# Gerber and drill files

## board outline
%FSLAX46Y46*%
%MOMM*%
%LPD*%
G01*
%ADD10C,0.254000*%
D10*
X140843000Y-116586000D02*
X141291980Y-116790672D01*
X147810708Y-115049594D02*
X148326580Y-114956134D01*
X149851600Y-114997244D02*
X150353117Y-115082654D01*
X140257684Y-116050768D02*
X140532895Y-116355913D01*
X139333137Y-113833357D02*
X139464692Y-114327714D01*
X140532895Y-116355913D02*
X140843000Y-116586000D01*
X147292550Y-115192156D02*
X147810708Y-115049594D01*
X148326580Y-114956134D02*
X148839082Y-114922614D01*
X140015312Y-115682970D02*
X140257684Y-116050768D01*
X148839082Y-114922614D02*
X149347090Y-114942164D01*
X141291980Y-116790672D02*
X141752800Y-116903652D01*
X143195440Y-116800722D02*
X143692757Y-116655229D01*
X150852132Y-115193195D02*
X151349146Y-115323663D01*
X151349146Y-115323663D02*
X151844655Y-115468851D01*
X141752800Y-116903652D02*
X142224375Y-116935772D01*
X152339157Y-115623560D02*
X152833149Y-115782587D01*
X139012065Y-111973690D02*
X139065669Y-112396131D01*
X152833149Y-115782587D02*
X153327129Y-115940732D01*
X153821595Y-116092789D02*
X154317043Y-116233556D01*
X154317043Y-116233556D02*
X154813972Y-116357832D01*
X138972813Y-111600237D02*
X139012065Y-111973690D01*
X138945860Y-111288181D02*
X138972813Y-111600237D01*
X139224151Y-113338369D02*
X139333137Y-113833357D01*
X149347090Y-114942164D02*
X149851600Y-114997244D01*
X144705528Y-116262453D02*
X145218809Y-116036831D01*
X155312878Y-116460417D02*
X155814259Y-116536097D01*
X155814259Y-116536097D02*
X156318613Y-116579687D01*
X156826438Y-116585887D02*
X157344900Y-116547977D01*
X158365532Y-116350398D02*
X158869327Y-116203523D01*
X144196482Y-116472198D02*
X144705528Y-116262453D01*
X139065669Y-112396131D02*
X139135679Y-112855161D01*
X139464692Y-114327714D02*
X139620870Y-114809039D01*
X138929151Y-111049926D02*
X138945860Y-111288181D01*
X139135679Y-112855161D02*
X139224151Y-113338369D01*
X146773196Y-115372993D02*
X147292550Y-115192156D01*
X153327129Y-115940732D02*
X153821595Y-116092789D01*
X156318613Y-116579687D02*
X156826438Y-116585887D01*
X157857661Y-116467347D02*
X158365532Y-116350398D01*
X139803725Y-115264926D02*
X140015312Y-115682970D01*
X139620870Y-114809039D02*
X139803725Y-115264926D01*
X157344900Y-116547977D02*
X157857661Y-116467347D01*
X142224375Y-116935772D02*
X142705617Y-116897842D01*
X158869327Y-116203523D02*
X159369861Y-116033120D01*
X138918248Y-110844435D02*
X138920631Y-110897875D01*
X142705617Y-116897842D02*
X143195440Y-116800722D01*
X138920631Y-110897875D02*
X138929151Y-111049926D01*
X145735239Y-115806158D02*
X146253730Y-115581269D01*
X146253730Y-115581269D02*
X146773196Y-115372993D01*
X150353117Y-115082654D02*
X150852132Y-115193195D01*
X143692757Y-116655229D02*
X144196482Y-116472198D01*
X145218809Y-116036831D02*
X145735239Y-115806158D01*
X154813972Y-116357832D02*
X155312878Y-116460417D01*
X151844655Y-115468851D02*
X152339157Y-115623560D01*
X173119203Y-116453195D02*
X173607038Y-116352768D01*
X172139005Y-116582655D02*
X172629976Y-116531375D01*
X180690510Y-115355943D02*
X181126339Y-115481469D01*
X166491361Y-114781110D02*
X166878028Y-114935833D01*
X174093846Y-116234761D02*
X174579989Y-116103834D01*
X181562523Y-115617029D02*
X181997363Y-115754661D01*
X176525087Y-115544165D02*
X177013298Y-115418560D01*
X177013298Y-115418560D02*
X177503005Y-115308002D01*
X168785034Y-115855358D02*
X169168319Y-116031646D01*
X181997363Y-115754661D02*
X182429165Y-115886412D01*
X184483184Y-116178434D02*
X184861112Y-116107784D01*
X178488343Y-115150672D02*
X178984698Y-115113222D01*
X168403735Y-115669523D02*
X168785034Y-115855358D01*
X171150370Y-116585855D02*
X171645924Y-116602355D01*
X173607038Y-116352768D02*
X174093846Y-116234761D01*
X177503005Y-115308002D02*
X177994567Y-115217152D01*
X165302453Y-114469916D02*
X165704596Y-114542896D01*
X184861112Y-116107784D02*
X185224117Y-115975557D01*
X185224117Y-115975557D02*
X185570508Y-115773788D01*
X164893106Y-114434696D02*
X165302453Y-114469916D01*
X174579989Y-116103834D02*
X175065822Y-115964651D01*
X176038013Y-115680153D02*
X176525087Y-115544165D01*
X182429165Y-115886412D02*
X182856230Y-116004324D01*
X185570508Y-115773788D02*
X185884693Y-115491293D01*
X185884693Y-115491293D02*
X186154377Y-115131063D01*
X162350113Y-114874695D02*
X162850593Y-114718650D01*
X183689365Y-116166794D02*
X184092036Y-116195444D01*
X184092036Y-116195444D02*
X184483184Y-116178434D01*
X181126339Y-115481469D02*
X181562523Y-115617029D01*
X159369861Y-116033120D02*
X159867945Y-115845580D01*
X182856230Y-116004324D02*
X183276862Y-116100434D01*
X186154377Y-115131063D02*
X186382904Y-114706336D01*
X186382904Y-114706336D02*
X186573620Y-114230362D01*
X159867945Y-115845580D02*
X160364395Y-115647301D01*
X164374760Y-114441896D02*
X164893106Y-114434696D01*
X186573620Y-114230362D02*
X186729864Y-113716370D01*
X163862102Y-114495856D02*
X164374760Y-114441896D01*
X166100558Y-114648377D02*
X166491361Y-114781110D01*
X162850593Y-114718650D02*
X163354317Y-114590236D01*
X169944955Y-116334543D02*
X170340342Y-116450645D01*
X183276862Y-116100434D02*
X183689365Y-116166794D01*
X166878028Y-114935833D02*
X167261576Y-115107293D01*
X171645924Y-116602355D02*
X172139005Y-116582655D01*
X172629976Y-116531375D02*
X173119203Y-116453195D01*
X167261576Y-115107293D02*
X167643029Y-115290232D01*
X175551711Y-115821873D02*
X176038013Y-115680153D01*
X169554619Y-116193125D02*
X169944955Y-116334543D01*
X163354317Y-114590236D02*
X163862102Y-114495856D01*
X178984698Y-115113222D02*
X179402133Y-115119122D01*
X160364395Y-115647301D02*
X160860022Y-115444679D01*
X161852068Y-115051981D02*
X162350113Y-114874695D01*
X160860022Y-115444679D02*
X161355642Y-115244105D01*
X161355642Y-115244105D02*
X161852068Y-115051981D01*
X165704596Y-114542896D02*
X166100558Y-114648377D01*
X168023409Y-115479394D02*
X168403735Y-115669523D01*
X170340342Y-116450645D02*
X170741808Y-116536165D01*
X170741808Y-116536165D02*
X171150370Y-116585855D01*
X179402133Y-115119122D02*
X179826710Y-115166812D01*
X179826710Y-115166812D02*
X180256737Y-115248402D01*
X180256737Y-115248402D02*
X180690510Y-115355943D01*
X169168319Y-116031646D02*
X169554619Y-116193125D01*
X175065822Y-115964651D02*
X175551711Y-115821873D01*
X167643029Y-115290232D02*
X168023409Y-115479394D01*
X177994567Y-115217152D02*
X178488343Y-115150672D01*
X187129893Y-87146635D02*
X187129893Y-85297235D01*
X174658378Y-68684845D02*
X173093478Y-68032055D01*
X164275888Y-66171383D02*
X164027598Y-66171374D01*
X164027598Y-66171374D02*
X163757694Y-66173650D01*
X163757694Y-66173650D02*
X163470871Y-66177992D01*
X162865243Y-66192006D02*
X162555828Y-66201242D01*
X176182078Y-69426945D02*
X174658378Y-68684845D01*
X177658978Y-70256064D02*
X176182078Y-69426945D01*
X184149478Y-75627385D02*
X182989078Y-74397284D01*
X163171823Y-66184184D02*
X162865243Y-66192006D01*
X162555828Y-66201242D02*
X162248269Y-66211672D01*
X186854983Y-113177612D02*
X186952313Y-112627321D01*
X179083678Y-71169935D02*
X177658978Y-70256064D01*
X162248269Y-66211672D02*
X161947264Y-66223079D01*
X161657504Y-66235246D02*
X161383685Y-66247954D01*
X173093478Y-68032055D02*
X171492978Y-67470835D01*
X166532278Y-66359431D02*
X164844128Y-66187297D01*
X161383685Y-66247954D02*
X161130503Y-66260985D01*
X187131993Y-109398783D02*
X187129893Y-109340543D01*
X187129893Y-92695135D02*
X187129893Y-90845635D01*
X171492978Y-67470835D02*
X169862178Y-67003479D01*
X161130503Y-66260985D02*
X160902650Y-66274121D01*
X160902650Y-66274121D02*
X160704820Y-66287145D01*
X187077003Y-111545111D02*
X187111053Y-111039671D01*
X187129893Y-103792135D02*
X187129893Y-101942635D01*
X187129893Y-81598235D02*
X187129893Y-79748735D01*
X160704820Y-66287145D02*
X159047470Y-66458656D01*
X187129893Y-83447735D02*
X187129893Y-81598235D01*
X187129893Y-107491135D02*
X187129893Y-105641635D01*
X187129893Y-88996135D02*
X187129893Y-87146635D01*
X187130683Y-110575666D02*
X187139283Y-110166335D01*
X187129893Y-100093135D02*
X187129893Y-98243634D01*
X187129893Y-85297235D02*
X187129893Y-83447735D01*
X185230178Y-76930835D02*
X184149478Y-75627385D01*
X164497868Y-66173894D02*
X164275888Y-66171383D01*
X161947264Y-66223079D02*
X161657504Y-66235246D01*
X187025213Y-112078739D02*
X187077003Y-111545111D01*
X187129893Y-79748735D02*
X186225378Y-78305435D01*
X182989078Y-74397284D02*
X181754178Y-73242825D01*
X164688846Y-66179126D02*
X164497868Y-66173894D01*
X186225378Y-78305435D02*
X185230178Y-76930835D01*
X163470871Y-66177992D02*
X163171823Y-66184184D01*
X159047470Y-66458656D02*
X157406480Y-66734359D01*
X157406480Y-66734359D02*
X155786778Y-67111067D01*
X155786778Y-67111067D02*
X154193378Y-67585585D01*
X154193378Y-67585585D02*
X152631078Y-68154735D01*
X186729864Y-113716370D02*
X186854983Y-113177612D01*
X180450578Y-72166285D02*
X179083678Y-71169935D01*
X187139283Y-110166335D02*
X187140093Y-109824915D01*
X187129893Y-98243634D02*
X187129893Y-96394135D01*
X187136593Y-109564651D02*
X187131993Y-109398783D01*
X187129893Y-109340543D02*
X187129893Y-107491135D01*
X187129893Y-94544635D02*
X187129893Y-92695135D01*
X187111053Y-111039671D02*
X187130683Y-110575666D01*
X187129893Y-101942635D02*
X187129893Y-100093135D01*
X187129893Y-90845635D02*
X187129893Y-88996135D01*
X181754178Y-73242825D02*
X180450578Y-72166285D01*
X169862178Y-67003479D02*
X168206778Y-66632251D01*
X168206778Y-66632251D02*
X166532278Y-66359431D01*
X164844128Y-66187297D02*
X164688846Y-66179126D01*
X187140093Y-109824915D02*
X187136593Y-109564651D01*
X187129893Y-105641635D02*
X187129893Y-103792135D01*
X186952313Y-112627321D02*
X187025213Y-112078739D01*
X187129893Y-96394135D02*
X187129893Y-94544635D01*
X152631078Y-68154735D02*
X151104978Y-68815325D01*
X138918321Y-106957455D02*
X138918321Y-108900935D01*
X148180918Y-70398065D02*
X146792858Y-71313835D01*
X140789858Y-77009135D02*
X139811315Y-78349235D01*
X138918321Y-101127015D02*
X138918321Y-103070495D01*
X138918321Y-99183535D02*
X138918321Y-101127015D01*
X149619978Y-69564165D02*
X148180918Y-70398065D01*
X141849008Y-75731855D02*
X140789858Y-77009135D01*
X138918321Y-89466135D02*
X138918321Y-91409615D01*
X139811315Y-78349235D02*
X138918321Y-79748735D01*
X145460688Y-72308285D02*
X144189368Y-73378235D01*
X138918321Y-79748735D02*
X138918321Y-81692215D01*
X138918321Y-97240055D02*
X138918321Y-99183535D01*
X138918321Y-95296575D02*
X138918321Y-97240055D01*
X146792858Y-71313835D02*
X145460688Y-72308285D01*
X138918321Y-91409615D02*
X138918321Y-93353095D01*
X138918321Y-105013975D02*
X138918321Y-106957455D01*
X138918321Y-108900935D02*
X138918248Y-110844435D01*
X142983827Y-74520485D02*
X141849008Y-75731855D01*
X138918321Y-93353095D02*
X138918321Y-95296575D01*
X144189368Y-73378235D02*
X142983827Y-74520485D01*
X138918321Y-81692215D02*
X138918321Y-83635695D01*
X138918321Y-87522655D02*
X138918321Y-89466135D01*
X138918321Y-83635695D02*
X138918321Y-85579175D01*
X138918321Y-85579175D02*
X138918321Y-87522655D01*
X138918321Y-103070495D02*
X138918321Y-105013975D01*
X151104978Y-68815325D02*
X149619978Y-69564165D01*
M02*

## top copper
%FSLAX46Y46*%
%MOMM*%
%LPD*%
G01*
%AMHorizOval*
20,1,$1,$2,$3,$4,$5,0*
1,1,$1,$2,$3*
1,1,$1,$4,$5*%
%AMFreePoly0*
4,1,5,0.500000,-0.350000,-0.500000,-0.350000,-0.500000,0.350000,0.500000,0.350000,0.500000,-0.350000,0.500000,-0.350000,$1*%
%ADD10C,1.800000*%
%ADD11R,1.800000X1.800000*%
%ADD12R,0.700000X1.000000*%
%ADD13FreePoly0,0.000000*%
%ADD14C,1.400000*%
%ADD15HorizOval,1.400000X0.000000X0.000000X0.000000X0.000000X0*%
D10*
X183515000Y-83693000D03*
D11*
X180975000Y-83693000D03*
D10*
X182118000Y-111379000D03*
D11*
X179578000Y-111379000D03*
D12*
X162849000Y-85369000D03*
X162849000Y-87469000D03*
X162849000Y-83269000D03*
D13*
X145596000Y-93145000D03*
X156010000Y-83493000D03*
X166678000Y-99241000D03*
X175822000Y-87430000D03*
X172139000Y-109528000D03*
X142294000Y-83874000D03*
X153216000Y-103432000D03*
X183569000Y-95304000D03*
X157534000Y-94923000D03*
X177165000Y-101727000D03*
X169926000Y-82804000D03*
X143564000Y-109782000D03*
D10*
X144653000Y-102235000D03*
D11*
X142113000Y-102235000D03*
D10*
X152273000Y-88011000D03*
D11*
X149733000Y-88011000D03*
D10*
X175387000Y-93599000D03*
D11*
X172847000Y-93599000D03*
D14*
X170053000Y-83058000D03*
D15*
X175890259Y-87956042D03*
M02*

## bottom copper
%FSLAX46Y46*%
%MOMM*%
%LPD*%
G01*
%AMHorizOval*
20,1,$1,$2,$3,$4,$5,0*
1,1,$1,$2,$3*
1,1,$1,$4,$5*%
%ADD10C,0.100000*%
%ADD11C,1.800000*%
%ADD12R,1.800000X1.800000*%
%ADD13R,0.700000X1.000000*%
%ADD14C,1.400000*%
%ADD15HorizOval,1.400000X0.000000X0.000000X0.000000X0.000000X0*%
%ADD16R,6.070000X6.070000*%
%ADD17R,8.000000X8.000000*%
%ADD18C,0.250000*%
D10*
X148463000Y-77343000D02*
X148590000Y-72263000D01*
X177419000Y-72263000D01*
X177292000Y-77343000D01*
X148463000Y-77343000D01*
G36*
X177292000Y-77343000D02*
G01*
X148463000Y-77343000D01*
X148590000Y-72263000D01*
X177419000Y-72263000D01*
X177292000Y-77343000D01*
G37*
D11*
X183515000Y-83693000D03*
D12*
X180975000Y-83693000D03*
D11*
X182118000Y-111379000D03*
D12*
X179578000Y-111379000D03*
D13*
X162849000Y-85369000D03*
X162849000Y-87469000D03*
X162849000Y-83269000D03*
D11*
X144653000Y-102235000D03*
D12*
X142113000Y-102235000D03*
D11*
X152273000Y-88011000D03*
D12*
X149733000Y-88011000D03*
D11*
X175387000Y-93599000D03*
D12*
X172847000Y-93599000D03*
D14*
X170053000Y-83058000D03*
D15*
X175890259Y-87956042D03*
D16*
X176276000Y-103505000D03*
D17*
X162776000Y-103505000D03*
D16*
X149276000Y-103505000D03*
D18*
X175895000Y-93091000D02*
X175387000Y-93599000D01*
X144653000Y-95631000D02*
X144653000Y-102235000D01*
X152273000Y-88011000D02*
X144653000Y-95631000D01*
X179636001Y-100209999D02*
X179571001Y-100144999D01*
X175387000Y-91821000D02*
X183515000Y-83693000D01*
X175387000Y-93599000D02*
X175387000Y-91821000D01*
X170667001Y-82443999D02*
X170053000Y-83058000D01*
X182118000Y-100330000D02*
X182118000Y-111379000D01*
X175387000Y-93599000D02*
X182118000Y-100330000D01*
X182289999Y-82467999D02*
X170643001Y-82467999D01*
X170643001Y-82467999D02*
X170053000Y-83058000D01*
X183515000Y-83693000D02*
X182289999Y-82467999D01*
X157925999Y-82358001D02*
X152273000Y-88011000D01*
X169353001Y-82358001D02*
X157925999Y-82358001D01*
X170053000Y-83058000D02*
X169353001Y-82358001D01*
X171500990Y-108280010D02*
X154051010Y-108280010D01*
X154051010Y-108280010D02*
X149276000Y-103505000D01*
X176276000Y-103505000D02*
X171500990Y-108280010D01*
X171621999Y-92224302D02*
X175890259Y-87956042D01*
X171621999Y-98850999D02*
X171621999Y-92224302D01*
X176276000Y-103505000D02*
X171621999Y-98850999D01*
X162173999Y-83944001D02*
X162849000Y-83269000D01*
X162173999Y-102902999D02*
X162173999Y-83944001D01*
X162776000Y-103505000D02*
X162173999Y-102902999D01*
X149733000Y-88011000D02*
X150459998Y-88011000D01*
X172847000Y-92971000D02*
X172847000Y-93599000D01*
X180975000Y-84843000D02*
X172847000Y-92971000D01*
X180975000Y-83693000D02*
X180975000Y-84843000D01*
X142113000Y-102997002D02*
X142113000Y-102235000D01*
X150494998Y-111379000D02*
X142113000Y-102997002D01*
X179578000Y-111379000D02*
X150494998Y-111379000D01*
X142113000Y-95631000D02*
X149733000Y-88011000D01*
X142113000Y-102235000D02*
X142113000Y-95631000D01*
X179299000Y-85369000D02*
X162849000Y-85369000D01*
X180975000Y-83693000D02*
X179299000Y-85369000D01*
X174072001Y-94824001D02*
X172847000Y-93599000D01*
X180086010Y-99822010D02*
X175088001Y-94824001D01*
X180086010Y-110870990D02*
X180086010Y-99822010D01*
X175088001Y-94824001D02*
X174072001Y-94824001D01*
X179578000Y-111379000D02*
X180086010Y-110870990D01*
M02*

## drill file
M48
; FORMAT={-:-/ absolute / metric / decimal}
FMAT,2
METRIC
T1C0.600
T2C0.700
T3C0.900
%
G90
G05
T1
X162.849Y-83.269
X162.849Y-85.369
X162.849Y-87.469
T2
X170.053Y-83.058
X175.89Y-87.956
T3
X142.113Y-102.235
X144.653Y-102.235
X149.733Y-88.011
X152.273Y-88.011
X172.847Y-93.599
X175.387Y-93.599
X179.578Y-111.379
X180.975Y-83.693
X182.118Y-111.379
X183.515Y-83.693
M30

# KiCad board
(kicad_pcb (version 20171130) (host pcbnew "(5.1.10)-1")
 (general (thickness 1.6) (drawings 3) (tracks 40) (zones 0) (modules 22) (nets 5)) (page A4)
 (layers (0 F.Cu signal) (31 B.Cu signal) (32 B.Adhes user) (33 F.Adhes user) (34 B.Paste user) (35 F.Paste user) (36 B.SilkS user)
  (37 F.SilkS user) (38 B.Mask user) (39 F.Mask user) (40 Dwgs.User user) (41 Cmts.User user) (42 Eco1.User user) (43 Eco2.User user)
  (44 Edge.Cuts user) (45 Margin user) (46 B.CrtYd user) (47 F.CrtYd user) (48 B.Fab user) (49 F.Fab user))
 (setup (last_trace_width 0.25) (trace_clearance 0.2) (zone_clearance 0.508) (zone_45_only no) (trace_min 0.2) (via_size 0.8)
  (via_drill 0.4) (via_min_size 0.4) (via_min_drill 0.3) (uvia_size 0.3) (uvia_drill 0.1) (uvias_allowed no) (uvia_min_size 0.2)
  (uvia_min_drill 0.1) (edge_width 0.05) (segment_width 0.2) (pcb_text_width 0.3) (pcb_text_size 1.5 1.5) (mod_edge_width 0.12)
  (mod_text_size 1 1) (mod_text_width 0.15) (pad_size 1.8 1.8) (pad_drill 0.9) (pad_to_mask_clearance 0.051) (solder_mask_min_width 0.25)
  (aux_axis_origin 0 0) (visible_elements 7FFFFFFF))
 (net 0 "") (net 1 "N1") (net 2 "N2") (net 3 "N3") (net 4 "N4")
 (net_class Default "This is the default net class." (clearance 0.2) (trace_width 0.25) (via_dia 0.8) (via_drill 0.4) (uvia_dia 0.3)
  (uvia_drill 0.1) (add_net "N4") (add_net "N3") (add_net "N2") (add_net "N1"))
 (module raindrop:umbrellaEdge (layer F.Cu) (at 162.687 92.456)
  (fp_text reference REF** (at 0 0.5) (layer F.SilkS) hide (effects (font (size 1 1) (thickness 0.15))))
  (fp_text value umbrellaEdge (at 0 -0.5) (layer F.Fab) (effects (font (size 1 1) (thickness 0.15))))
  (fp_line (start -21.844 24.13) (end -21.39502 24.334672) (layer Edge.Cuts) (width 0.254))
  (fp_line (start -14.876292 22.593594) (end -14.36042 22.500134) (layer Edge.Cuts) (width 0.254))
  (fp_line (start -12.8354 22.541244) (end -12.333883 22.626654) (layer Edge.Cuts) (width 0.254))
  (fp_line (start -22.429316 23.594768) (end -22.154105 23.899913) (layer Edge.Cuts) (width 0.254))
  (fp_line (start -23.353863 21.377357) (end -23.222308 21.871714) (layer Edge.Cuts) (width 0.254))
  (fp_line (start -22.154105 23.899913) (end -21.844 24.13) (layer Edge.Cuts) (width 0.254))
  (fp_line (start -15.39445 22.736156) (end -14.876292 22.593594) (layer Edge.Cuts) (width 0.254))
  (fp_line (start -14.36042 22.500134) (end -13.847918 22.466614) (layer Edge.Cuts) (width 0.254))
  (fp_line (start -22.671688 23.22697) (end -22.429316 23.594768) (layer Edge.Cuts) (width 0.254))
  (fp_line (start -13.847918 22.466614) (end -13.33991 22.486164) (layer Edge.Cuts) (width 0.254))
  (fp_line (start -21.39502 24.334672) (end -20.9342 24.447652) (layer Edge.Cuts) (width 0.254))
  (fp_line (start -19.49156 24.344722) (end -18.994243 24.199229) (layer Edge.Cuts) (width 0.254))
  (fp_line (start -11.834868 22.737195) (end -11.337854 22.867663) (layer Edge.Cuts) (width 0.254))
  (fp_line (start -11.337854 22.867663) (end -10.842345 23.012851) (layer Edge.Cuts) (width 0.254))
  (fp_line (start -20.9342 24.447652) (end -20.462625 24.479772) (layer Edge.Cuts) (width 0.254))
  (fp_line (start -10.347843 23.16756) (end -9.853851 23.326587) (layer Edge.Cuts) (width 0.254))
  (fp_line (start -23.674935 19.51769) (end -23.621331 19.940131) (layer Edge.Cuts) (width 0.254))
  (fp_line (start -9.853851 23.326587) (end -9.359871 23.484732) (layer Edge.Cuts) (width 0.254))
  (fp_line (start -8.865405 23.636789) (end -8.369957 23.777556) (layer Edge.Cuts) (width 0.254))
  (fp_line (start -8.369957 23.777556) (end -7.873028 23.901832) (layer Edge.Cuts) (width 0.254))
  (fp_line (start -23.714187 19.144237) (end -23.674935 19.51769) (layer Edge.Cuts) (width 0.254))
  (fp_line (start -23.74114 18.832181) (end -23.714187 19.144237) (layer Edge.Cuts) (width 0.254))
  (fp_line (start -23.462849 20.882369) (end -23.353863 21.377357) (layer Edge.Cuts) (width 0.254))
  (fp_line (start -13.33991 22.486164) (end -12.8354 22.541244) (layer Edge.Cuts) (width 0.254))
  (fp_line (start -17.981472 23.806453) (end -17.468191 23.580831) (layer Edge.Cuts) (width 0.254))
  (fp_line (start -7.374122 24.004417) (end -6.872741 24.080097) (layer Edge.Cuts) (width 0.254))
  (fp_line (start -6.872741 24.080097) (end -6.368387 24.123687) (layer Edge.Cuts) (width 0.254))
  (fp_line (start -5.860562 24.129887) (end -5.3421 24.091977) (layer Edge.Cuts) (width 0.254))
  (fp_line (start -4.321468 23.894398) (end -3.817673 23.747523) (layer Edge.Cuts) (width 0.254))
  (fp_line (start -18.490518 24.016198) (end -17.981472 23.806453) (layer Edge.Cuts) (width 0.254))
  (fp_line (start -23.621331 19.940131) (end -23.551321 20.399161) (layer Edge.Cuts) (width 0.254))
  (fp_line (start -23.222308 21.871714) (end -23.06613 22.353039) (layer Edge.Cuts) (width 0.254))
  (fp_line (start -23.757849 18.593926) (end -23.74114 18.832181) (layer Edge.Cuts) (width 0.254))
  (fp_line (start -23.551321 20.399161) (end -23.462849 20.882369) (layer Edge.Cuts) (width 0.254))
  (fp_line (start -15.913804 22.916993) (end -15.39445 22.736156) (layer Edge.Cuts) (width 0.254))
  (fp_line (start -9.359871 23.484732) (end -8.865405 23.636789) (layer Edge.Cuts) (width 0.254))
  (fp_line (start -6.368387 24.123687) (end -5.860562 24.129887) (layer Edge.Cuts) (width 0.254))
  (fp_line (start -4.829339 24.011347) (end -4.321468 23.894398) (layer Edge.Cuts) (width 0.254))
  (fp_line (start -22.883275 22.808926) (end -22.671688 23.22697) (layer Edge.Cuts) (width 0.254))
  (fp_line (start -23.06613 22.353039) (end -22.883275 22.808926) (layer Edge.Cuts) (width 0.254))
  (fp_line (start -5.3421 24.091977) (end -4.829339 24.011347) (layer Edge.Cuts) (width 0.254))
  (fp_line (start -20.462625 24.479772) (end -19.981383 24.441842) (layer Edge.Cuts) (width 0.254))
  (fp_line (start -3.817673 23.747523) (end -3.317139 23.57712) (layer Edge.Cuts) (width 0.254))
  (fp_line (start -23.768752 18.388435) (end -23.766369 18.441875) (layer Edge.Cuts) (width 0.254))
  (fp_line (start -19.981383 24.441842) (end -19.49156 24.344722) (layer Edge.Cuts) (width 0.254))
  (fp_line (start -23.766369 18.441875) (end -23.757849 18.593926) (layer Edge.Cuts) (width 0.254))
  (fp_line (start -16.951761 23.350158) (end -16.43327 23.125269) (layer Edge.Cuts) (width 0.254))
  (fp_line (start -16.43327 23.125269) (end -15.913804 22.916993) (layer Edge.Cuts) (width 0.254))
  (fp_line (start -12.333883 22.626654) (end -11.834868 22.737195) (layer Edge.Cuts) (width 0.254))
  (fp_line (start -18.994243 24.199229) (end -18.490518 24.016198) (layer Edge.Cuts) (width 0.254))
  (fp_line (start -17.468191 23.580831) (end -16.951761 23.350158) (layer Edge.Cuts) (width 0.254))
  (fp_line (start -7.873028 23.901832) (end -7.374122 24.004417) (layer Edge.Cuts) (width 0.254))
  (fp_line (start -10.842345 23.012851) (end -10.347843 23.16756) (layer Edge.Cuts) (width 0.254))
  (fp_line (start 10.432203 23.997195) (end 10.920038 23.896768) (layer Edge.Cuts) (width 0.254))
  (fp_line (start 9.452005 24.126655) (end 9.942976 24.075375) (layer Edge.Cuts) (width 0.254))
  (fp_line (start 18.00351 22.899943) (end 18.439339 23.025469) (layer Edge.Cuts) (width 0.254))
  (fp_line (start 3.804361 22.32511) (end 4.191028 22.479833) (layer Edge.Cuts) (width 0.254))
  (fp_line (start 11.406846 23.778761) (end 11.892989 23.647834) (layer Edge.Cuts) (width 0.254))
  (fp_line (start 18.875523 23.161029) (end 19.310363 23.298661) (layer Edge.Cuts) (width 0.254))
  (fp_line (start 13.838087 23.088165) (end 14.326298 22.96256) (layer Edge.Cuts) (width 0.254))
  (fp_line (start 14.326298 22.96256) (end 14.816005 22.852002) (layer Edge.Cuts) (width 0.254))
  (fp_line (start 6.098034 23.399358) (end 6.481319 23.575646) (layer Edge.Cuts) (width 0.254))
  (fp_line (start 19.310363 23.298661) (end 19.742165 23.430412) (layer Edge.Cuts) (width 0.254))
  (fp_line (start 21.796184 23.722434) (end 22.174112 23.651784) (layer Edge.Cuts) (width 0.254))
  (fp_line (start 15.801343 22.694672) (end 16.297698 22.657222) (layer Edge.Cuts) (width 0.254))
  (fp_line (start 5.716735 23.213523) (end 6.098034 23.399358) (layer Edge.Cuts) (width 0.254))
  (fp_line (start 8.46337 24.129855) (end 8.958924 24.146355) (layer Edge.Cuts) (width 0.254))
  (fp_line (start 10.920038 23.896768) (end 11.406846 23.778761) (layer Edge.Cuts) (width 0.254))
  (fp_line (start 14.816005 22.852002) (end 15.307567 22.761152) (layer Edge.Cuts) (width 0.254))
  (fp_line (start 2.615453 22.013916) (end 3.017596 22.086896) (layer Edge.Cuts) (width 0.254))
  (fp_line (start 22.174112 23.651784) (end 22.537117 23.519557) (layer Edge.Cuts) (width 0.254))
  (fp_line (start 22.537117 23.519557) (end 22.883508 23.317788) (layer Edge.Cuts) (width 0.254))
  (fp_line (start 2.206106 21.978696) (end 2.615453 22.013916) (layer Edge.Cuts) (width 0.254))
  (fp_line (start 11.892989 23.647834) (end 12.378822 23.508651) (layer Edge.Cuts) (width 0.254))
  (fp_line (start 13.351013 23.224153) (end 13.838087 23.088165) (layer Edge.Cuts) (width 0.254))
  (fp_line (start 19.742165 23.430412) (end 20.16923 23.548324) (layer Edge.Cuts) (width 0.254))
  (fp_line (start 22.883508 23.317788) (end 23.197693 23.035293) (layer Edge.Cuts) (width 0.254))
  (fp_line (start 23.197693 23.035293) (end 23.467377 22.675063) (layer Edge.Cuts) (width 0.254))
  (fp_line (start -0.336887 22.418695) (end 0.163593 22.26265) (layer Edge.Cuts) (width 0.254))
  (fp_line (start 21.002365 23.710794) (end 21.405036 23.739444) (layer Edge.Cuts) (width 0.254))
  (fp_line (start 21.405036 23.739444) (end 21.796184 23.722434) (layer Edge.Cuts) (width 0.254))
  (fp_line (start 18.439339 23.025469) (end 18.875523 23.161029) (layer Edge.Cuts) (width 0.254))
  (fp_line (start -3.317139 23.57712) (end -2.819055 23.38958) (layer Edge.Cuts) (width 0.254))
  (fp_line (start 20.16923 23.548324) (end 20.589862 23.644434) (layer Edge.Cuts) (width 0.254))
  (fp_line (start 23.467377 22.675063) (end 23.695904 22.250336) (layer Edge.Cuts) (width 0.254))
  (fp_line (start 23.695904 22.250336) (end 23.88662 21.774362) (layer Edge.Cuts) (width 0.254))
  (fp_line (start -2.819055 23.38958) (end -2.322605 23.191301) (layer Edge.Cuts) (width 0.254))
  (fp_line (start 1.68776 21.985896) (end 2.206106 21.978696) (layer Edge.Cuts) (width 0.254))
  (fp_line (start 23.88662 21.774362) (end 24.042864 21.26037) (layer Edge.Cuts) (width 0.254))
  (fp_line (start 1.175102 22.039856) (end 1.68776 21.985896) (layer Edge.Cuts) (width 0.254))
  (fp_line (start 3.413558 22.192377) (end 3.804361 22.32511) (layer Edge.Cuts) (width 0.254))
  (fp_line (start 0.163593 22.26265) (end 0.667317 22.134236) (layer Edge.Cuts) (width 0.254))
  (fp_line (start 7.257955 23.878543) (end 7.653342 23.994645) (layer Edge.Cuts) (width 0.254))
  (fp_line (start 20.589862 23.644434) (end 21.002365 23.710794) (layer Edge.Cuts) (width 0.254))
  (fp_line (start 4.191028 22.479833) (end 4.574576 22.651293) (layer Edge.Cuts) (width 0.254))
  (fp_line (start 8.958924 24.146355) (end 9.452005 24.126655) (layer Edge.Cuts) (width 0.254))
  (fp_line (start 9.942976 24.075375) (end 10.432203 23.997195) (layer Edge.Cuts) (width 0.254))
  (fp_line (start 4.574576 22.651293) (end 4.956029 22.834232) (layer Edge.Cuts) (width 0.254))
  (fp_line (start 12.864711 23.365873) (end 13.351013 23.224153) (layer Edge.Cuts) (width 0.254))
  (fp_line (start 6.867619 23.737125) (end 7.257955 23.878543) (layer Edge.Cuts) (width 0.254))
  (fp_line (start 0.667317 22.134236) (end 1.175102 22.039856) (layer Edge.Cuts) (width 0.254))
  (fp_line (start 16.297698 22.657222) (end 16.715133 22.663122) (layer Edge.Cuts) (width 0.254))
  (fp_line (start -2.322605 23.191301) (end -1.826978 22.988679) (layer Edge.Cuts) (width 0.254))
  (fp_line (start -0.834932 22.595981) (end -0.336887 22.418695) (layer Edge.Cuts) (width 0.254))
  (fp_line (start -1.826978 22.988679) (end -1.331358 22.788105) (layer Edge.Cuts) (width 0.254))
  (fp_line (start -1.331358 22.788105) (end -0.834932 22.595981) (layer Edge.Cuts) (width 0.254))
  (fp_line (start 3.017596 22.086896) (end 3.413558 22.192377) (layer Edge.Cuts) (width 0.254))
  (fp_line (start 5.336409 23.023394) (end 5.716735 23.213523) (layer Edge.Cuts) (width 0.254))
  (fp_line (start 7.653342 23.994645) (end 8.054808 24.080165) (layer Edge.Cuts) (width 0.254))
  (fp_line (start 8.054808 24.080165) (end 8.46337 24.129855) (layer Edge.Cuts) (width 0.254))
  (fp_line (start 16.715133 22.663122) (end 17.13971 22.710812) (layer Edge.Cuts) (width 0.254))
  (fp_line (start 17.13971 22.710812) (end 17.569737 22.792402) (layer Edge.Cuts) (width 0.254))
  (fp_line (start 17.569737 22.792402) (end 18.00351 22.899943) (layer Edge.Cuts) (width 0.254))
  (fp_line (start 6.481319 23.575646) (end 6.867619 23.737125) (layer Edge.Cuts) (width 0.254))
  (fp_line (start 12.378822 23.508651) (end 12.864711 23.365873) (layer Edge.Cuts) (width 0.254))
  (fp_line (start 4.956029 22.834232) (end 5.336409 23.023394) (layer Edge.Cuts) (width 0.254))
  (fp_line (start 15.307567 22.761152) (end 15.801343 22.694672) (layer Edge.Cuts) (width 0.254))
  (fp_line (start 24.442893 -5.309365) (end 24.442893 -7.158765) (layer Edge.Cuts) (width 0.254))
  (fp_line (start 11.971378 -23.771155) (end 10.406478 -24.423945) (layer Edge.Cuts) (width 0.254))
  (fp_line (start 1.588888 -26.284617) (end 1.340598 -26.284626) (layer Edge.Cuts) (width 0.254))
  (fp_line (start 1.340598 -26.284626) (end 1.070694 -26.28235) (layer Edge.Cuts) (width 0.254))
  (fp_line (start 1.070694 -26.28235) (end 0.783871 -26.278008) (layer Edge.Cuts) (width 0.254))
  (fp_line (start 0.178243 -26.263994) (end -0.131172 -26.254758) (layer Edge.Cuts) (width 0.254))
  (fp_line (start 13.495078 -23.029055) (end 11.971378 -23.771155) (layer Edge.Cuts) (width 0.254))
  (fp_line (start 14.971978 -22.199936) (end 13.495078 -23.029055) (layer Edge.Cuts) (width 0.254))
  (fp_line (start 21.462478 -16.828615) (end 20.302078 -18.058716) (layer Edge.Cuts) (width 0.254))
  (fp_line (start 0.484823 -26.271816) (end 0.178243 -26.263994) (layer Edge.Cuts) (width 0.254))
  (fp_line (start -0.131172 -26.254758) (end -0.438731 -26.244328) (layer Edge.Cuts) (width 0.254))
  (fp_line (start 24.167983 20.721612) (end 24.265313 20.171321) (layer Edge.Cuts) (width 0.254))
  (fp_line (start 16.396678 -21.286065) (end 14.971978 -22.199936) (layer Edge.Cuts) (width 0.254))
  (fp_line (start -0.438731 -26.244328) (end -0.739736 -26.232921) (layer Edge.Cuts) (width 0.254))
  (fp_line (start -1.029496 -26.220754) (end -1.303315 -26.208046) (layer Edge.Cuts) (width 0.254))
  (fp_line (start 10.406478 -24.423945) (end 8.805978 -24.985165) (layer Edge.Cuts) (width 0.254))
  (fp_line (start 3.845278 -26.096569) (end 2.157128 -26.268703) (layer Edge.Cuts) (width 0.254))
  (fp_line (start -1.303315 -26.208046) (end -1.556497 -26.195015) (layer Edge.Cuts) (width 0.254))
  (fp_line (start 24.444993 16.942783) (end 24.442893 16.884543) (layer Edge.Cuts) (width 0.254))
  (fp_line (start 24.442893 0.239135) (end 24.442893 -1.610365) (layer Edge.Cuts) (width 0.254))
  (fp_line (start 8.805978 -24.985165) (end 7.175178 -25.452521) (layer Edge.Cuts) (width 0.254))
  (fp_line (start -1.556497 -26.195015) (end -1.78435 -26.181879) (layer Edge.Cuts) (width 0.254))
  (fp_line (start -1.78435 -26.181879) (end -1.98218 -26.168855) (layer Edge.Cuts) (width 0.254))
  (fp_line (start 24.390003 19.089111) (end 24.424053 18.583671) (layer Edge.Cuts) (width 0.254))
  (fp_line (start 24.442893 11.336135) (end 24.442893 9.486635) (layer Edge.Cuts) (width 0.254))
  (fp_line (start 24.442893 -10.857765) (end 24.442893 -12.707265) (layer Edge.Cuts) (width 0.254))
  (fp_line (start -1.98218 -26.168855) (end -3.63953 -25.997344) (layer Edge.Cuts) (width 0.254))
  (fp_line (start 24.442893 -9.008265) (end 24.442893 -10.857765) (layer Edge.Cuts) (width 0.254))
  (fp_line (start 24.442893 15.035135) (end 24.442893 13.185635) (layer Edge.Cuts) (width 0.254))
  (fp_line (start 24.442893 -3.459865) (end 24.442893 -5.309365) (layer Edge.Cuts) (width 0.254))
  (fp_line (start 24.443683 18.119666) (end 24.452283 17.710335) (layer Edge.Cuts) (width 0.254))
  (fp_line (start 24.442893 7.637135) (end 24.442893 5.787634) (layer Edge.Cuts) (width 0.254))
  (fp_line (start 24.442893 -7.158765) (end 24.442893 -9.008265) (layer Edge.Cuts) (width 0.254))
  (fp_line (start 22.543178 -15.525165) (end 21.462478 -16.828615) (layer Edge.Cuts) (width 0.254))
  (fp_line (start 1.810868 -26.282106) (end 1.588888 -26.284617) (layer Edge.Cuts) (width 0.254))
  (fp_line (start -0.739736 -26.232921) (end -1.029496 -26.220754) (layer Edge.Cuts) (width 0.254))
  (fp_line (start 24.338213 19.622739) (end 24.390003 19.089111) (layer Edge.Cuts) (width 0.254))
  (fp_line (start 24.442893 -12.707265) (end 23.538378 -14.150565) (layer Edge.Cuts) (width 0.254))
  (fp_line (start 20.302078 -18.058716) (end 19.067178 -19.213175) (layer Edge.Cuts) (width 0.254))
  (fp_line (start 2.001846 -26.276874) (end 1.810868 -26.282106) (layer Edge.Cuts) (width 0.254))
  (fp_line (start 23.538378 -14.150565) (end 22.543178 -15.525165) (layer Edge.Cuts) (width 0.254))
  (fp_line (start 0.783871 -26.278008) (end 0.484823 -26.271816) (layer Edge.Cuts) (width 0.254))
  (fp_line (start -3.63953 -25.997344) (end -5.28052 -25.721641) (layer Edge.Cuts) (width 0.254))
  (fp_line (start -5.28052 -25.721641) (end -6.900222 -25.344933) (layer Edge.Cuts) (width 0.254))
  (fp_line (start -6.900222 -25.344933) (end -8.493622 -24.870415) (layer Edge.Cuts) (width 0.254))
  (fp_line (start -8.493622 -24.870415) (end -10.055922 -24.301265) (layer Edge.Cuts) (width 0.254))
  (fp_line (start 24.042864 21.26037) (end 24.167983 20.721612) (layer Edge.Cuts) (width 0.254))
  (fp_line (start 17.763578 -20.289715) (end 16.396678 -21.286065) (layer Edge.Cuts) (width 0.254))
  (fp_line (start 24.452283 17.710335) (end 24.453093 17.368915) (layer Edge.Cuts) (width 0.254))
  (fp_line (start 24.442893 5.787634) (end 24.442893 3.938135) (layer Edge.Cuts) (width 0.254))
  (fp_line (start 24.449593 17.108651) (end 24.444993 16.942783) (layer Edge.Cuts) (width 0.254))
  (fp_line (start 24.442893 16.884543) (end 24.442893 15.035135) (layer Edge.Cuts) (width 0.254))
  (fp_line (start 24.442893 2.088635) (end 24.442893 0.239135) (layer Edge.Cuts) (width 0.254))
  (fp_line (start 24.424053 18.583671) (end 24.443683 18.119666) (layer Edge.Cuts) (width 0.254))
  (fp_line (start 24.442893 9.486635) (end 24.442893 7.637135) (layer Edge.Cuts) (width 0.254))
  (fp_line (start 24.442893 -1.610365) (end 24.442893 -3.459865) (layer Edge.Cuts) (width 0.254))
  (fp_line (start 19.067178 -19.213175) (end 17.763578 -20.289715) (layer Edge.Cuts) (width 0.254))
  (fp_line (start 7.175178 -25.452521) (end 5.519778 -25.823749) (layer Edge.Cuts) (width 0.254))
  (fp_line (start 5.519778 -25.823749) (end 3.845278 -26.096569) (layer Edge.Cuts) (width 0.254))
  (fp_line (start 2.157128 -26.268703) (end 2.001846 -26.276874) (layer Edge.Cuts) (width 0.254))
  (fp_line (start 24.453093 17.368915) (end 24.449593 17.108651) (layer Edge.Cuts) (width 0.254))
  (fp_line (start 24.442893 13.185635) (end 24.442893 11.336135) (layer Edge.Cuts) (width 0.254))
  (fp_line (start 24.265313 20.171321) (end 24.338213 19.622739) (layer Edge.Cuts) (width 0.254))
  (fp_line (start 24.442893 3.938135) (end 24.442893 2.088635) (layer Edge.Cuts) (width 0.254))
  (fp_line (start -10.055922 -24.301265) (end -11.582022 -23.640675) (layer Edge.Cuts) (width 0.254))
  (fp_line (start -23.768679 14.501455) (end -23.768679 16.444935) (layer Edge.Cuts) (width 0.254))
  (fp_line (start -14.506082 -22.057935) (end -15.894142 -21.142165) (layer Edge.Cuts) (width 0.254))
  (fp_line (start -21.897142 -15.446865) (end -22.875685 -14.106765) (layer Edge.Cuts) (width 0.254))
  (fp_line (start -23.768679 8.671015) (end -23.768679 10.614495) (layer Edge.Cuts) (width 0.254))
  (fp_line (start -23.768679 6.727535) (end -23.768679 8.671015) (layer Edge.Cuts) (width 0.254))
  (fp_line (start -13.067022 -22.891835) (end -14.506082 -22.057935) (layer Edge.Cuts) (width 0.254))
  (fp_line (start -20.837992 -16.724145) (end -21.897142 -15.446865) (layer Edge.Cuts) (width 0.254))
  (fp_line (start -23.768679 -2.989865) (end -23.768679 -1.046385) (layer Edge.Cuts) (width 0.254))
  (fp_line (start -22.875685 -14.106765) (end -23.768679 -12.707265) (layer Edge.Cuts) (width 0.254))
  (fp_line (start -17.226312 -20.147715) (end -18.497632 -19.077765) (layer Edge.Cuts) (width 0.254))
  (fp_line (start -23.768679 -12.707265) (end -23.768679 -10.763785) (layer Edge.Cuts) (width 0.254))
  (fp_line (start -23.768679 4.784055) (end -23.768679 6.727535) (layer Edge.Cuts) (width 0.254))
  (fp_line (start -23.768679 2.840575) (end -23.768679 4.784055) (layer Edge.Cuts) (width 0.254))
  (fp_line (start -15.894142 -21.142165) (end -17.226312 -20.147715) (layer Edge.Cuts) (width 0.254))
  (fp_line (start -23.768679 -1.046385) (end -23.768679 0.897095) (layer Edge.Cuts) (width 0.254))
  (fp_line (start -23.768679 12.557975) (end -23.768679 14.501455) (layer Edge.Cuts) (width 0.254))
  (fp_line (start -23.768679 16.444935) (end -23.768752 18.388435) (layer Edge.Cuts) (width 0.254))
  (fp_line (start -19.703173 -17.935515) (end -20.837992 -16.724145) (layer Edge.Cuts) (width 0.254))
  (fp_line (start -23.768679 0.897095) (end -23.768679 2.840575) (layer Edge.Cuts) (width 0.254))
  (fp_line (start -18.497632 -19.077765) (end -19.703173 -17.935515) (layer Edge.Cuts) (width 0.254))
  (fp_line (start -23.768679 -10.763785) (end -23.768679 -8.820305) (layer Edge.Cuts) (width 0.254))
  (fp_line (start -23.768679 -4.933345) (end -23.768679 -2.989865) (layer Edge.Cuts) (width 0.254))
  (fp_line (start -23.768679 -8.820305) (end -23.768679 -6.876825) (layer Edge.Cuts) (width 0.254))
  (fp_line (start -23.768679 -6.876825) (end -23.768679 -4.933345) (layer Edge.Cuts) (width 0.254))
  (fp_line (start -23.768679 10.614495) (end -23.768679 12.557975) (layer Edge.Cuts) (width 0.254))
  (fp_line (start -11.582022 -23.640675) (end -13.067022 -22.891835) (layer Edge.Cuts) (width 0.254)))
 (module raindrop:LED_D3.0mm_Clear (layer F.Cu) (at 180.975 83.693)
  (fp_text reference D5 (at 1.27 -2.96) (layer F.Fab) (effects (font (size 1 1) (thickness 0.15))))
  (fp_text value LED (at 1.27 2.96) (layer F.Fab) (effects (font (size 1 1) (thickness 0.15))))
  (pad 2 thru_hole circle (at 2.54 0) (size 1.8 1.8) (drill 0.9) (layers *.Cu *.Mask) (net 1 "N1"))
  (pad 1 thru_hole rect (at 0 0) (size 1.8 1.8) (drill 0.9) (layers *.Cu *.Mask) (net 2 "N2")))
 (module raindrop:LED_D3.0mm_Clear (layer F.Cu) (at 179.578 111.379)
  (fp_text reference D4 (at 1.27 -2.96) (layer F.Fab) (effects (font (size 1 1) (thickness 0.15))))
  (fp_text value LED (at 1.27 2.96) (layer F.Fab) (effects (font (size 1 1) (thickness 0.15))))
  (pad 2 thru_hole circle (at 2.54 0) (size 1.8 1.8) (drill 0.9) (layers *.Cu *.Mask) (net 1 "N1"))
  (pad 1 thru_hole rect (at 0 0) (size 1.8 1.8) (drill 0.9) (layers *.Cu *.Mask) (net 2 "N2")))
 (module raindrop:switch (layer B.Cu) (at 163.449 82.169 270)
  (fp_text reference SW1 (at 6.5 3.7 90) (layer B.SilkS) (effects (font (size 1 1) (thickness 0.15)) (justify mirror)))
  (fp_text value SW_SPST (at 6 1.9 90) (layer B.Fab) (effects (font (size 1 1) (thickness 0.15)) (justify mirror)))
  (pad 2 thru_hole rect (at 3.2 0.6 270) (size 1 0.7) (drill 0.6) (layers *.Cu *.Mask) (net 2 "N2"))
  (pad 3 thru_hole rect (at 5.3 0.6 270) (size 1 0.7) (drill 0.6) (layers *.Cu *.Mask))
  (pad 1 thru_hole rect (at 1.1 0.6 270) (size 1 0.7) (drill 0.6) (layers *.Cu *.Mask) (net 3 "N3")))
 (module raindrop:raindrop (layer F.Cu) (at 145.796 93.345)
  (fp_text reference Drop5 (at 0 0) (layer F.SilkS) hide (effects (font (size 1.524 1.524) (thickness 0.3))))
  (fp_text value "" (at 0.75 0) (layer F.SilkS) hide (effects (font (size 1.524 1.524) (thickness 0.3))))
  (pad 1 smd custom (at -0.2 -0.2) (size 1 0.7) (layers F.Cu F.Paste F.Mask) (zone_connect 0) (options (clearance outline) (anchor rect))
   (primitives)))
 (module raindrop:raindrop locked (layer F.Cu) (at 156.21 83.693)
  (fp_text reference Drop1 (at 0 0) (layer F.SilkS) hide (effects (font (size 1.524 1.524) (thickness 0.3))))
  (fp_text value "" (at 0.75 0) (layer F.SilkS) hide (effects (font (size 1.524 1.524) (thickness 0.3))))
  (pad 1 smd custom (at -0.2 -0.2) (size 1 0.7) (layers F.Cu F.Paste F.Mask) (zone_connect 0) (options (clearance outline) (anchor rect))
   (primitives)))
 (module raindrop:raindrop (layer F.Cu) (at 166.878 99.441)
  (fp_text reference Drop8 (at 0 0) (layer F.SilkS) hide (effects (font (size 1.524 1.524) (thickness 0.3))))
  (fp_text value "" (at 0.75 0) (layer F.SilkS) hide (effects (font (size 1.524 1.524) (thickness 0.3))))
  (pad 1 smd custom (at -0.2 -0.2) (size 1 0.7) (layers F.Cu F.Paste F.Mask) (zone_connect 0) (options (clearance outline) (anchor rect))
   (primitives)))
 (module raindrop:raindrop (layer F.Cu) (at 176.022 87.63)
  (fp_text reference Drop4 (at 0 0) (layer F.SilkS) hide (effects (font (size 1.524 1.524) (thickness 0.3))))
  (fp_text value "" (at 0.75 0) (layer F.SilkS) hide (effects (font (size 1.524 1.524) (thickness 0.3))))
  (pad 1 smd custom (at -0.2 -0.2) (size 1 0.7) (layers F.Cu F.Paste F.Mask) (zone_connect 0) (options (clearance outline) (anchor rect))
   (primitives)))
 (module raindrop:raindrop (layer F.Cu) (at 172.339 109.728)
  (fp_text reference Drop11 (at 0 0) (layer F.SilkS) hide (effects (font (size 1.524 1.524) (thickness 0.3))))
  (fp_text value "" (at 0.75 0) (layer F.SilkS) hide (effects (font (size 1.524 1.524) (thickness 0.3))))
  (pad 1 smd custom (at -0.2 -0.2) (size 1 0.7) (layers F.Cu F.Paste F.Mask) (zone_connect 0) (options (clearance outline) (anchor rect))
   (primitives)))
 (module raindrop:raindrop (layer F.Cu) (at 142.494 84.074)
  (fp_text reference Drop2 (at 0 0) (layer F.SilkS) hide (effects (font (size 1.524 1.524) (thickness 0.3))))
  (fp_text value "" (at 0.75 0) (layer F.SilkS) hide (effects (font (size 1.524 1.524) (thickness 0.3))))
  (pad 1 smd custom (at -0.2 -0.2) (size 1 0.7) (layers F.Cu F.Paste F.Mask) (zone_connect 0) (options (clearance outline) (anchor rect))
   (primitives)))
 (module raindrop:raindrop (layer F.Cu) (at 153.416 103.632)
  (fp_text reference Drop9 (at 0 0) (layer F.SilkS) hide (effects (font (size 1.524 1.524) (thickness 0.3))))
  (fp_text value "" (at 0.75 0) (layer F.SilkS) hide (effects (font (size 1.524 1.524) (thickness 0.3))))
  (pad 1 smd custom (at -0.2 -0.2) (size 1 0.7) (layers F.Cu F.Paste F.Mask) (zone_connect 0) (options (clearance outline) (anchor rect))
   (primitives)))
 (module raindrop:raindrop (layer F.Cu) (at 183.769 95.504)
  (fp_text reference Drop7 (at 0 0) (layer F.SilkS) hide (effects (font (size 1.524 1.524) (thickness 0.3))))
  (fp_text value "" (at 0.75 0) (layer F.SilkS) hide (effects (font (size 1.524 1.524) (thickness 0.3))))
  (pad 1 smd custom (at -0.2 -0.2) (size 1 0.7) (layers F.Cu F.Paste F.Mask) (zone_connect 0) (options (clearance outline) (anchor rect))
   (primitives)))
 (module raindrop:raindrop (layer F.Cu) (at 157.734 95.123)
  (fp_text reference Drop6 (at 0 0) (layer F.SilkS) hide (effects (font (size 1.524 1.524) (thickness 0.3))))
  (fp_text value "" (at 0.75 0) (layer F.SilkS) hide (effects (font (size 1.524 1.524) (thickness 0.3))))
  (pad 1 smd custom (at -0.2 -0.2) (size 1 0.7) (layers F.Cu F.Paste F.Mask) (zone_connect 0) (options (clearance outline) (anchor rect))
   (primitives)))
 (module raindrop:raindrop (layer F.Cu) (at 177.365 101.927)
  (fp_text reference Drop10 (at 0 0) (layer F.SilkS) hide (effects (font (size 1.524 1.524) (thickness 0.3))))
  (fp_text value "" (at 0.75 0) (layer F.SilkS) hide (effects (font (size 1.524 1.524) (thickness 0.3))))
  (pad 1 smd custom (at -0.2 -0.2) (size 1 0.7) (layers F.Cu F.Paste F.Mask) (zone_connect 0) (options (clearance outline) (anchor rect))
   (primitives)))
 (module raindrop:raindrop (layer F.Cu) (at 170.126 83.004)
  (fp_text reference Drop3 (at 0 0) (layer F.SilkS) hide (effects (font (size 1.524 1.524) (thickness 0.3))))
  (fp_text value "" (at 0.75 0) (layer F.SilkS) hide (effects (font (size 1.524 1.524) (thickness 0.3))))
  (pad 1 smd custom (at -0.2 -0.2) (size 1 0.7) (layers F.Cu F.Paste F.Mask) (zone_connect 0) (options (clearance outline) (anchor rect))
   (primitives)))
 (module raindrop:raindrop (layer F.Cu) (at 143.764 109.982)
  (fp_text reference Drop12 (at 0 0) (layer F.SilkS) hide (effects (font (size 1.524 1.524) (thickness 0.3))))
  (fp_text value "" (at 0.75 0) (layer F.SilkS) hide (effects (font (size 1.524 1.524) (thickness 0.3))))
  (pad 1 smd custom (at -0.2 -0.2) (size 1 0.7) (layers F.Cu F.Paste F.Mask) (zone_connect 0) (options (clearance outline) (anchor rect))
   (primitives)))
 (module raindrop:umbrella (layer F.Cu) (at 163.068 91.567)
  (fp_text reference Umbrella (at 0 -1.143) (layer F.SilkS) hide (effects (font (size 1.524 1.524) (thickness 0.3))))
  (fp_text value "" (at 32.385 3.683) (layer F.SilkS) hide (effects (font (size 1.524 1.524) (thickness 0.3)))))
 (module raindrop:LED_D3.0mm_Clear (layer F.Cu) (at 142.113 102.235)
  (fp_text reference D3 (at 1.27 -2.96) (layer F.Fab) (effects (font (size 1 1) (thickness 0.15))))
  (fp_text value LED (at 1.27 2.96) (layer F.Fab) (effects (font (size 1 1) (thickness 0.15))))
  (pad 2 thru_hole circle (at 2.54 0) (size 1.8 1.8) (drill 0.9) (layers *.Cu *.Mask) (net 1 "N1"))
  (pad 1 thru_hole rect (at 0 0) (size 1.8 1.8) (drill 0.9) (layers *.Cu *.Mask) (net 2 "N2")))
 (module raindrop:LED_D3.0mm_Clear (layer F.Cu) (at 149.733 88.011)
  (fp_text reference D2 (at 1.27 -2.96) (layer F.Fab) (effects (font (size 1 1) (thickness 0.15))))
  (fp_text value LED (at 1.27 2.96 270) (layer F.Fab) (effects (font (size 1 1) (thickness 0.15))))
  (pad 2 thru_hole circle (at 2.54 0) (size 1.8 1.8) (drill 0.9) (layers *.Cu *.Mask) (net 1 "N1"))
  (pad 1 thru_hole rect (at 0 0) (size 1.8 1.8) (drill 0.9) (layers *.Cu *.Mask) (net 2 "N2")))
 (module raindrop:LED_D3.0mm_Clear (layer F.Cu) (at 172.847 93.599)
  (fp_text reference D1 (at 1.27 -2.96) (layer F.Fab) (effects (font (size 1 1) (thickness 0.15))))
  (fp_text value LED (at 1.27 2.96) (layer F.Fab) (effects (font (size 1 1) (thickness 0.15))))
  (pad 2 thru_hole circle (at 2.54 0) (size 1.8 1.8) (drill 0.9) (layers *.Cu *.Mask) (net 1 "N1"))
  (pad 1 thru_hole rect (at 0 0) (size 1.8 1.8) (drill 0.9) (layers *.Cu *.Mask) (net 2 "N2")))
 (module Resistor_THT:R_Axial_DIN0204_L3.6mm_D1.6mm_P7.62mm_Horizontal (layer B.Cu) (at 170.053 83.058 320)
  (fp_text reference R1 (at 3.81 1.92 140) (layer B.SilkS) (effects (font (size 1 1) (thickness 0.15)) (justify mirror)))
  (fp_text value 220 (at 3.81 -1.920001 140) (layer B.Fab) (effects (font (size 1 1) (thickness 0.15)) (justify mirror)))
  (pad 1 thru_hole circle (at 0 0 320) (size 1.4 1.4) (drill 0.7) (layers *.Cu *.Mask) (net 1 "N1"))
  (pad 2 thru_hole oval (at 7.62 0 320) (size 1.4 1.4) (drill 0.7) (layers *.Cu *.Mask) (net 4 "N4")))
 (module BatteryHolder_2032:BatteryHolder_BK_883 (layer B.Cu) (at 162.776 102.905)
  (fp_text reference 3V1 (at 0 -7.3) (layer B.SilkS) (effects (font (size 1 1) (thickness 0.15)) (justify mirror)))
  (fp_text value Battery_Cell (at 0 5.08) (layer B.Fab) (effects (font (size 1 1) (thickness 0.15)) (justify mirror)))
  (pad 1 smd rect (at 13.5 0.6) (size 6.07 6.07) (layers B.Cu B.Paste B.Mask) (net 4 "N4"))
  (pad 2 smd rect (at 0 0.6) (size 8 8) (layers B.Cu B.Paste B.Mask) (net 3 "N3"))
  (pad 1 smd rect (at -13.5 0.6) (size 6.07 6.07) (layers B.Cu B.Paste B.Mask) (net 4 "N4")))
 (gr_poly (pts (xy 148.463 77.343) (xy 148.59 72.263) (xy 177.419 72.263) (xy 177.292 77.343)) (layer B.Cu) (width 0.1))
 (segment (start 175.895 93.091) (end 175.387 93.599) (width 0.25) (layer B.Cu) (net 1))
 (segment (start 144.653 95.631) (end 144.653 102.235) (width 0.25) (layer B.Cu) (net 1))
 (segment (start 152.273 88.011) (end 144.653 95.631) (width 0.25) (layer B.Cu) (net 1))
 (segment (start 179.636001 100.209999) (end 179.571001 100.144999) (width 0.25) (layer B.Cu) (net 1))
 (segment (start 175.387 91.821) (end 183.515 83.693) (width 0.25) (layer B.Cu) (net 1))
 (segment (start 175.387 93.599) (end 175.387 91.821) (width 0.25) (layer B.Cu) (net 1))
 (segment (start 170.667001 82.443999) (end 170.053 83.058) (width 0.25) (layer B.Cu) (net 1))
 (segment (start 182.118 100.33) (end 182.118 111.379) (width 0.25) (layer B.Cu) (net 1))
 (segment (start 175.387 93.599) (end 182.118 100.33) (width 0.25) (layer B.Cu) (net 1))
 (segment (start 182.289999 82.467999) (end 170.643001 82.467999) (width 0.25) (layer B.Cu) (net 1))
 (segment (start 170.643001 82.467999) (end 170.053 83.058) (width 0.25) (layer B.Cu) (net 1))
 (segment (start 183.515 83.693) (end 182.289999 82.467999) (width 0.25) (layer B.Cu) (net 1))
 (segment (start 157.925999 82.358001) (end 152.273 88.011) (width 0.25) (layer B.Cu) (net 1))
 (segment (start 169.353001 82.358001) (end 157.925999 82.358001) (width 0.25) (layer B.Cu) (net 1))
 (segment (start 170.053 83.058) (end 169.353001 82.358001) (width 0.25) (layer B.Cu) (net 1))
 (segment (start 171.50099 108.28001) (end 154.05101 108.28001) (width 0.25) (layer B.Cu) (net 4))
 (segment (start 154.05101 108.28001) (end 149.276 103.505) (width 0.25) (layer B.Cu) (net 4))
 (segment (start 176.276 103.505) (end 171.50099 108.28001) (width 0.25) (layer B.Cu) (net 4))
 (segment (start 171.621999 92.224302) (end 175.890259 87.956042) (width 0.25) (layer B.Cu) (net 4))
 (segment (start 171.621999 98.850999) (end 171.621999 92.224302) (width 0.25) (layer B.Cu) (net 4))
 (segment (start 176.276 103.505) (end 171.621999 98.850999) (width 0.25) (layer B.Cu) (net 4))
 (segment (start 162.173999 83.944001) (end 162.849 83.269) (width 0.25) (layer B.Cu) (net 3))
 (segment (start 162.173999 102.902999) (end 162.173999 83.944001) (width 0.25) (layer B.Cu) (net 3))
 (segment (start 162.776 103.505) (end 162.173999 102.902999) (width 0.25) (layer B.Cu) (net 3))
 (segment (start 149.733 88.011) (end 150.459998 88.011) (width 0.25) (layer B.Cu) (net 2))
 (segment (start 172.847 92.971) (end 172.847 93.599) (width 0.25) (layer B.Cu) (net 2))
 (segment (start 180.975 84.843) (end 172.847 92.971) (width 0.25) (layer B.Cu) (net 2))
 (segment (start 180.975 83.693) (end 180.975 84.843) (width 0.25) (layer B.Cu) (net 2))
 (segment (start 142.113 102.997002) (end 142.113 102.235) (width 0.25) (layer B.Cu) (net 2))
 (segment (start 150.494998 111.379) (end 142.113 102.997002) (width 0.25) (layer B.Cu) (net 2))
 (segment (start 179.578 111.379) (end 150.494998 111.379) (width 0.25) (layer B.Cu) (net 2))
 (segment (start 142.113 95.631) (end 149.733 88.011) (width 0.25) (layer B.Cu) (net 2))
 (segment (start 142.113 102.235) (end 142.113 95.631) (width 0.25) (layer B.Cu) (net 2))
 (segment (start 179.299 85.369) (end 162.849 85.369) (width 0.25) (layer B.Cu) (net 2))
 (segment (start 180.975 83.693) (end 179.299 85.369) (width 0.25) (layer B.Cu) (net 2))
 (segment (start 174.072001 94.824001) (end 172.847 93.599) (width 0.25) (layer B.Cu) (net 2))
 (segment (start 180.08601 99.82201) (end 175.088001 94.824001) (width 0.25) (layer B.Cu) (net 2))
 (segment (start 180.08601 110.87099) (end 180.08601 99.82201) (width 0.25) (layer B.Cu) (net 2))
 (segment (start 175.088001 94.824001) (end 174.072001 94.824001) (width 0.25) (layer B.Cu) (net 2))
 (segment (start 179.578 111.379) (end 180.08601 110.87099) (width 0.25) (layer B.Cu) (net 2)))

